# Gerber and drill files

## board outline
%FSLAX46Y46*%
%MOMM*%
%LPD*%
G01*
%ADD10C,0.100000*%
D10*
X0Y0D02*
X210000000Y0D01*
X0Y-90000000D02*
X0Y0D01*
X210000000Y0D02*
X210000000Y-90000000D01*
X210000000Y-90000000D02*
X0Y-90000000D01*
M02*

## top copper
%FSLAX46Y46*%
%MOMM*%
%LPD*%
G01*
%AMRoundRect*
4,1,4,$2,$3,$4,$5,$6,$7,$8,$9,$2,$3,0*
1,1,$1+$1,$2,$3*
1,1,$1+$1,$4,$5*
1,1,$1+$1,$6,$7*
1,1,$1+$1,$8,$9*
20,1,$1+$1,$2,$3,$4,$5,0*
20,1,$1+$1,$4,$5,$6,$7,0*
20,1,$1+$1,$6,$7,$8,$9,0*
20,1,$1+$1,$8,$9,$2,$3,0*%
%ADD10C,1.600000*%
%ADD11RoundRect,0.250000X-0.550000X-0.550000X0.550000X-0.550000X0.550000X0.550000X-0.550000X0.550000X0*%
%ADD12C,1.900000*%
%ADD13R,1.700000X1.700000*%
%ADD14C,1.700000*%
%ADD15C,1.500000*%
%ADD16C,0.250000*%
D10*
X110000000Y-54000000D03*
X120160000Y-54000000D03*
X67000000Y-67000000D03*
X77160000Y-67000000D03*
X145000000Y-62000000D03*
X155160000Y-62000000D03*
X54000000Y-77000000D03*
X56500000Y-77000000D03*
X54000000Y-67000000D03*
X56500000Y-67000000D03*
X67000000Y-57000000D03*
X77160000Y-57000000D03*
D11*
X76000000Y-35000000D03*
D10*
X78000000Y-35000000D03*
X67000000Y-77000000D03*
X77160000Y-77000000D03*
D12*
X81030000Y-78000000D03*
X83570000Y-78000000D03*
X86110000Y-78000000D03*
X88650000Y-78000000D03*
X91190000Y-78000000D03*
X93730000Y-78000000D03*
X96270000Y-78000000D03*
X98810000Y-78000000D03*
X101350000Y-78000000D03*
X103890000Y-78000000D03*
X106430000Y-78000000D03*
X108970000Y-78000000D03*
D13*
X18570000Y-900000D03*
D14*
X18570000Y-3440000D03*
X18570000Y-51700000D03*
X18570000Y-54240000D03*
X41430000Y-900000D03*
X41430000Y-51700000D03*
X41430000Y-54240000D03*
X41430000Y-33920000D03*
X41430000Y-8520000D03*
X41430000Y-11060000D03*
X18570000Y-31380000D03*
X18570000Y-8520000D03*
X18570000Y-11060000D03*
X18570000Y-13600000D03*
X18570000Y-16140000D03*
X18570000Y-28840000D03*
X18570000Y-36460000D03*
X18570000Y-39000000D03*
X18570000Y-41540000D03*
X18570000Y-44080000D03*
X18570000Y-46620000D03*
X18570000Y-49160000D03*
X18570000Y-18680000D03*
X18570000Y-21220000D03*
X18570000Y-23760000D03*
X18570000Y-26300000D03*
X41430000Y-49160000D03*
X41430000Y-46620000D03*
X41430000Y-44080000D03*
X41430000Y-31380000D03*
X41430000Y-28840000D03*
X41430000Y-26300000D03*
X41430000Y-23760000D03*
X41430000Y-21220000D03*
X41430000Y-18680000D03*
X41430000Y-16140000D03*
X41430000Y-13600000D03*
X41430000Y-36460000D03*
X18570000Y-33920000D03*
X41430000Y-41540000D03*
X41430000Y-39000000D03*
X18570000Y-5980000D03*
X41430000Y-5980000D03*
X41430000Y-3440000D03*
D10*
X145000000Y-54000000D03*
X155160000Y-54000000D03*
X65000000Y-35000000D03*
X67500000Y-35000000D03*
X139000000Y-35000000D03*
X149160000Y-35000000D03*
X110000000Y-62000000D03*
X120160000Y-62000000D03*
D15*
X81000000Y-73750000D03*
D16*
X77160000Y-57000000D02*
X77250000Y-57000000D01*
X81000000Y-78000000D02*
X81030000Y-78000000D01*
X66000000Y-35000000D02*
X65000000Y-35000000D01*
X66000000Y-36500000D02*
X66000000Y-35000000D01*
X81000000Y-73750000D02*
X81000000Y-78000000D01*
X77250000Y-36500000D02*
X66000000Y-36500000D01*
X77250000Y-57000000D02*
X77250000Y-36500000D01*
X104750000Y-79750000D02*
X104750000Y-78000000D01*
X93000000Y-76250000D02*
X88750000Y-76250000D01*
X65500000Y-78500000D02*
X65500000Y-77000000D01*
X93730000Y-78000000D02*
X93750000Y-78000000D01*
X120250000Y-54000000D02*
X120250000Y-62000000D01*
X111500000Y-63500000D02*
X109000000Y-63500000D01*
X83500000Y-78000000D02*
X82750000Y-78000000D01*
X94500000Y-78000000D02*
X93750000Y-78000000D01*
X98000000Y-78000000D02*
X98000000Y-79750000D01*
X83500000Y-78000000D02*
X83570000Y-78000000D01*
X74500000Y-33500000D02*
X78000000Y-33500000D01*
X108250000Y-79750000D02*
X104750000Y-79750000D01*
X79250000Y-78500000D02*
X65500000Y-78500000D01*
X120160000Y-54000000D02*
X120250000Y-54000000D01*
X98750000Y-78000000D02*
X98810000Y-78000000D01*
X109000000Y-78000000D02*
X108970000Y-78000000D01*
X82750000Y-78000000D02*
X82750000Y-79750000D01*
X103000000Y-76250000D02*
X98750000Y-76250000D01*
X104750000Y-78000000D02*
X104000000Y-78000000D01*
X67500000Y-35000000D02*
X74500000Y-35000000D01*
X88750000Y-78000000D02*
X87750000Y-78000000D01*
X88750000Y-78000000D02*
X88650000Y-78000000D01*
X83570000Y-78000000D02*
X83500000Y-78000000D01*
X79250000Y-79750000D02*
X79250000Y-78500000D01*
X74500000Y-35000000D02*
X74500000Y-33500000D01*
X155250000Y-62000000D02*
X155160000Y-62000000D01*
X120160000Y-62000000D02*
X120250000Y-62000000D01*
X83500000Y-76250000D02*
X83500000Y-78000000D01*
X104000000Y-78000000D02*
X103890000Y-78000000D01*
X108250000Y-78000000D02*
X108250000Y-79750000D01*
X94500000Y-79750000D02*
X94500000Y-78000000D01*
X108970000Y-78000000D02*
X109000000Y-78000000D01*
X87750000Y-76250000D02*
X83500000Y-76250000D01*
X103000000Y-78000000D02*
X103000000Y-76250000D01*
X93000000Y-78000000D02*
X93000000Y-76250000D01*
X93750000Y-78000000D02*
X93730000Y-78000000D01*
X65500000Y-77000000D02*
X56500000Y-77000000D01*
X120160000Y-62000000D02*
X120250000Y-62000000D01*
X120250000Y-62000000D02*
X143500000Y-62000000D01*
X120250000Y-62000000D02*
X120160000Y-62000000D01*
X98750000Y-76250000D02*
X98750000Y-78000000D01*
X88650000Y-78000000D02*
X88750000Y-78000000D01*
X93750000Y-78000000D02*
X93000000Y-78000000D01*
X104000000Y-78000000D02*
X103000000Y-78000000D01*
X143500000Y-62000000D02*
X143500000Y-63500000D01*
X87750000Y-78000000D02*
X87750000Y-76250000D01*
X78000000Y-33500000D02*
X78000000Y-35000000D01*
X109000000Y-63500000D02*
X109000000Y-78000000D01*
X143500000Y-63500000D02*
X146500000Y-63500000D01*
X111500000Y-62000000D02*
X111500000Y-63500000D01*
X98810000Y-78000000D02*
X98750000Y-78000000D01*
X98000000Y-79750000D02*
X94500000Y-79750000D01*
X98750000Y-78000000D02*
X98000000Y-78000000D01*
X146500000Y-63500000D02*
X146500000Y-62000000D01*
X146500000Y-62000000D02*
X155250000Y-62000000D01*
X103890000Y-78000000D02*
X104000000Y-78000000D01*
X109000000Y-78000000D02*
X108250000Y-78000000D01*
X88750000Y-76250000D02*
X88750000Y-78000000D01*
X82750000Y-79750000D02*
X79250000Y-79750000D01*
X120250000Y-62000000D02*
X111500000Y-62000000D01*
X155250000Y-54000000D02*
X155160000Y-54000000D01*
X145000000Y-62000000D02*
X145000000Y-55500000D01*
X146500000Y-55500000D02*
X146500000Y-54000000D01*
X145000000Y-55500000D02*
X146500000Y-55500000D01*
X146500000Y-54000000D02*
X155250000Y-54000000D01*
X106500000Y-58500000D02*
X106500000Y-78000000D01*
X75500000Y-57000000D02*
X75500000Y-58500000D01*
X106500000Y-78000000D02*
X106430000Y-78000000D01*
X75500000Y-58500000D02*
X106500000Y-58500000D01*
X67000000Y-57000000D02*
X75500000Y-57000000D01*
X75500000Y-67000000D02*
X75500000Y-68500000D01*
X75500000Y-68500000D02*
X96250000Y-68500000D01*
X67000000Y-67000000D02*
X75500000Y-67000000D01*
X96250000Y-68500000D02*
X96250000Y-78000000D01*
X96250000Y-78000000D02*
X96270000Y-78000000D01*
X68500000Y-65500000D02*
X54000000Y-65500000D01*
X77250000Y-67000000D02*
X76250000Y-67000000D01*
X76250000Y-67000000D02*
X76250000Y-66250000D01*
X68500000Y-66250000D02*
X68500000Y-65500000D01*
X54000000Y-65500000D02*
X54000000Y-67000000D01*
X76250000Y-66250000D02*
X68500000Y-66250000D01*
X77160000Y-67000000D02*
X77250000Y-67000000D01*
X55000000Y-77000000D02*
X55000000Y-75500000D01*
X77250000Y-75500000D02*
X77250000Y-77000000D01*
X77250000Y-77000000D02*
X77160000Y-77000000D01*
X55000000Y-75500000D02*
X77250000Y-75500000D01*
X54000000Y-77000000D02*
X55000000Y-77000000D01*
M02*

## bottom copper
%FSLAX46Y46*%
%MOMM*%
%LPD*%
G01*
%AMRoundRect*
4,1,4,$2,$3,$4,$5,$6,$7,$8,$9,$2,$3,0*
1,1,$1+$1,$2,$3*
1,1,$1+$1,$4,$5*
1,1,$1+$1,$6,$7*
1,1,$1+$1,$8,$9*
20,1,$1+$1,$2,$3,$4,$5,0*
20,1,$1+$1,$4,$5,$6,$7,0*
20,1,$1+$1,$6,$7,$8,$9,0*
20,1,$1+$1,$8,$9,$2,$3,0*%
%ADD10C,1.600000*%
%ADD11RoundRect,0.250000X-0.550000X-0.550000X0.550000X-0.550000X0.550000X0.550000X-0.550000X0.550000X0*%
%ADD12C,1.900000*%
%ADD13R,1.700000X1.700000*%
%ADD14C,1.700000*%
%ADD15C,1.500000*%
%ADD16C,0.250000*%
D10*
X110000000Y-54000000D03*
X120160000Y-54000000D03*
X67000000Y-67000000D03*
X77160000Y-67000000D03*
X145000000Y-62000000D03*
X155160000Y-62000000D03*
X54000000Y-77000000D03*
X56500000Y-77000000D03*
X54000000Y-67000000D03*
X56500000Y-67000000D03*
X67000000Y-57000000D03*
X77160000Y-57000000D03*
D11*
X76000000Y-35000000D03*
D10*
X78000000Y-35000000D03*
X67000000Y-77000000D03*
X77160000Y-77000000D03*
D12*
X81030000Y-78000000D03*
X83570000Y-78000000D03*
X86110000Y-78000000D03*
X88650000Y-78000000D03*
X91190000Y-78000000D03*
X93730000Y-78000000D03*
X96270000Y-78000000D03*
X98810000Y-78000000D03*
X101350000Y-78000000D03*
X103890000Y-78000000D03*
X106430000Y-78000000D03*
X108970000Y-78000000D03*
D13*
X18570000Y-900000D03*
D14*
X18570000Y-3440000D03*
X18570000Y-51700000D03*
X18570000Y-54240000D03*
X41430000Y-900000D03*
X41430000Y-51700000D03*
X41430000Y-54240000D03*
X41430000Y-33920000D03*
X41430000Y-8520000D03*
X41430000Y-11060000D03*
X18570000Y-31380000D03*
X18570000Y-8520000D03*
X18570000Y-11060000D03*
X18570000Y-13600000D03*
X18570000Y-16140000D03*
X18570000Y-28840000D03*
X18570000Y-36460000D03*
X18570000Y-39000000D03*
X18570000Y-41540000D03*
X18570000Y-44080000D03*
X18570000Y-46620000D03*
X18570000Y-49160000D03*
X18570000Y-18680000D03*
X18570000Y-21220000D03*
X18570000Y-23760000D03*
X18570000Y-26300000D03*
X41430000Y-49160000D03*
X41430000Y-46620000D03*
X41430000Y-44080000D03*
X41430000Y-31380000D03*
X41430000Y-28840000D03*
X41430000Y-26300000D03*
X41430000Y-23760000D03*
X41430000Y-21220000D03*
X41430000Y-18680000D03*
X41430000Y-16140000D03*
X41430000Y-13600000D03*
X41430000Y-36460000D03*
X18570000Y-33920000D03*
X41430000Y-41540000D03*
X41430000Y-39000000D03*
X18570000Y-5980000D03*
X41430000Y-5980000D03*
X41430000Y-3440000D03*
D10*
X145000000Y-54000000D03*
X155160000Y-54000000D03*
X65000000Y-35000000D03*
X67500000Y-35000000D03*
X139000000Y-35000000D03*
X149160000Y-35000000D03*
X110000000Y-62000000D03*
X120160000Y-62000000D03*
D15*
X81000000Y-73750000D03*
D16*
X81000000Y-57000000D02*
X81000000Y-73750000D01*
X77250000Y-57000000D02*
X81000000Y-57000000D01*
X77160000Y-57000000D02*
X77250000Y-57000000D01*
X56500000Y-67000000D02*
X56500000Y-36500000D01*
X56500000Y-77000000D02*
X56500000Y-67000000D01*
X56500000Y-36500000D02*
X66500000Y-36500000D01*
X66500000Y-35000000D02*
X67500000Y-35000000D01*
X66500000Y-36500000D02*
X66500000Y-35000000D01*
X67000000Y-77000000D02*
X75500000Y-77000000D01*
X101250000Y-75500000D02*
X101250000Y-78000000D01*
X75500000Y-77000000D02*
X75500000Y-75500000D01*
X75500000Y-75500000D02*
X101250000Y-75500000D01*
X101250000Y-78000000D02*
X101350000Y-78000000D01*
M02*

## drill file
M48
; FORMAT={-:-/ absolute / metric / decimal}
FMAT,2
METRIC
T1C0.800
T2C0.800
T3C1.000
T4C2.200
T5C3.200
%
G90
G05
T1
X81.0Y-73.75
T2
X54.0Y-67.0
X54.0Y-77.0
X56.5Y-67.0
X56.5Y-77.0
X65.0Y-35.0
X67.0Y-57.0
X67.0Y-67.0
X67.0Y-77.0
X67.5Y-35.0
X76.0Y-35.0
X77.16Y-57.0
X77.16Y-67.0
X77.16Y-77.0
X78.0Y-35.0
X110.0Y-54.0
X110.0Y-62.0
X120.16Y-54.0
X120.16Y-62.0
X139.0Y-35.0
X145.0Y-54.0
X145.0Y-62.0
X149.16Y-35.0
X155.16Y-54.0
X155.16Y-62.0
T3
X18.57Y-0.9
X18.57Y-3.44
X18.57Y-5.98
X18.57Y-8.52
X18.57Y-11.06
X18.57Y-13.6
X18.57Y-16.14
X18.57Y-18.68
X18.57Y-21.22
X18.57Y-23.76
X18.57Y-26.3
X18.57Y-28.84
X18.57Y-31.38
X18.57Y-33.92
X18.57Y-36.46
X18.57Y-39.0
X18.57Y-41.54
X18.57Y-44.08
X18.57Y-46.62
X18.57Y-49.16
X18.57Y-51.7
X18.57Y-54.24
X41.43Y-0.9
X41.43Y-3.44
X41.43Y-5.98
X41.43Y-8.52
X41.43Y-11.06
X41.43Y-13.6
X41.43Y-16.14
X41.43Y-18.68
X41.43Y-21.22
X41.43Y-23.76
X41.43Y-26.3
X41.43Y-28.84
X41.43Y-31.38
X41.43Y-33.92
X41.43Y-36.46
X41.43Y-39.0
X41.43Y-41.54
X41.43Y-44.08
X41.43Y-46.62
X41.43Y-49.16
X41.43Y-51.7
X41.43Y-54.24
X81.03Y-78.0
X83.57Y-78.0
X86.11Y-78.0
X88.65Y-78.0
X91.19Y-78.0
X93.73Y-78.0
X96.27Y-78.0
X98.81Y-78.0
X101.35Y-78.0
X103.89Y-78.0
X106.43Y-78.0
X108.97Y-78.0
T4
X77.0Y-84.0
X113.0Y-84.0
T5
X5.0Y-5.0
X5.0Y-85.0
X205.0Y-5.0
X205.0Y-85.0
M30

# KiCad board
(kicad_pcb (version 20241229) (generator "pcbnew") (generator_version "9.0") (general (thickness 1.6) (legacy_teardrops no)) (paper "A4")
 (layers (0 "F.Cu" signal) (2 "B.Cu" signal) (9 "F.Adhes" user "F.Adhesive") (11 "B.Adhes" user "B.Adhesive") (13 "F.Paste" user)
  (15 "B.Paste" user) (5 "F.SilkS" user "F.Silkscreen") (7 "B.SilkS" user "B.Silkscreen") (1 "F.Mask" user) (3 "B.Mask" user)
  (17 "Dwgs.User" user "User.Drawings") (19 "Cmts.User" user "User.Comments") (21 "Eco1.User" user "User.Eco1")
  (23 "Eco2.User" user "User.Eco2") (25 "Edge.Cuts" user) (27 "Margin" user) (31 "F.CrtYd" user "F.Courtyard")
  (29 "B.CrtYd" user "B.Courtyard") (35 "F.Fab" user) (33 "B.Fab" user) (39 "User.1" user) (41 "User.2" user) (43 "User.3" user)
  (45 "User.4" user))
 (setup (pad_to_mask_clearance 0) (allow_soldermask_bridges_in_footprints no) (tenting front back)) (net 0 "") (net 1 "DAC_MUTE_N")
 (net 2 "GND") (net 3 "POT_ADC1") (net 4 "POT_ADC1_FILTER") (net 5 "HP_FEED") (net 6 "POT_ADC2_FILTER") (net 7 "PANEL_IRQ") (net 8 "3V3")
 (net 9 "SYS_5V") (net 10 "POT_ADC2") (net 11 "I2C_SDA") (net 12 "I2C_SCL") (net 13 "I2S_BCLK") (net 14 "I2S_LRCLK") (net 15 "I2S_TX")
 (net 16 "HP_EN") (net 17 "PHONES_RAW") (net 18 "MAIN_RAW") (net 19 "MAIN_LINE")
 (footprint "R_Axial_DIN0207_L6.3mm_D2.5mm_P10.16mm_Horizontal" (layer "F.Cu") (at 110 54)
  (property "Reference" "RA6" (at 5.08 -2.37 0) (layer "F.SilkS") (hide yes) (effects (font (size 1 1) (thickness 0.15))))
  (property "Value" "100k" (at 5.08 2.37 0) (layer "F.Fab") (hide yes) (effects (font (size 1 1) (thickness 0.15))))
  (pad "1" thru_hole circle (at 0 0) (size 1.6 1.6) (drill 0.8) (layers "*.Cu" "*.Mask") (remove_unused_layers no) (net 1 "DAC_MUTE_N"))
  (pad "2" thru_hole circle (at 10.16 0) (size 1.6 1.6) (drill 0.8) (layers "*.Cu" "*.Mask") (remove_unused_layers no) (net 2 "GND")))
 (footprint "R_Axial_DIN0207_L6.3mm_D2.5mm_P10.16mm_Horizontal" (layer "F.Cu") (at 67 67)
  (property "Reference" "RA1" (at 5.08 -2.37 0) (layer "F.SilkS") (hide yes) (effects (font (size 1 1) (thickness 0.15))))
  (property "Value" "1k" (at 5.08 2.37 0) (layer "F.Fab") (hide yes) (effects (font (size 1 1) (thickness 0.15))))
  (pad "1" thru_hole circle (at 0 0) (size 1.6 1.6) (drill 0.8) (layers "*.Cu" "*.Mask") (remove_unused_layers no) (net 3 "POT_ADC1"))
  (pad "2" thru_hole circle (at 10.16 0) (size 1.6 1.6) (drill 0.8) (layers "*.Cu" "*.Mask") (remove_unused_layers no)
   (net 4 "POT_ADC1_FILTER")))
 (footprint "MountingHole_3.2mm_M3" (layer "F.Cu") (at 5 5)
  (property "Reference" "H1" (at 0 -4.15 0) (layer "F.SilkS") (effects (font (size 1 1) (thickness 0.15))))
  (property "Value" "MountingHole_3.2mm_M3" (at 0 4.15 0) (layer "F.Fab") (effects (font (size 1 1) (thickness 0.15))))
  (pad "" np_thru_hole circle (at 0 0) (size 3.2 3.2) (drill 3.2) (layers "*.Cu" "*.Mask")))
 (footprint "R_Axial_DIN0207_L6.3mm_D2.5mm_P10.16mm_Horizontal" (layer "F.Cu") (at 145 62)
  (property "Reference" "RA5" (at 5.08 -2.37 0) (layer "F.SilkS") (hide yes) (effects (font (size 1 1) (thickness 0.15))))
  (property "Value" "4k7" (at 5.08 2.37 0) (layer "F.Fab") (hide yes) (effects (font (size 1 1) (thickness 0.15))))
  (pad "1" thru_hole circle (at 0 0) (size 1.6 1.6) (drill 0.8) (layers "*.Cu" "*.Mask") (remove_unused_layers no) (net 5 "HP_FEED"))
  (pad "2" thru_hole circle (at 10.16 0) (size 1.6 1.6) (drill 0.8) (layers "*.Cu" "*.Mask") (remove_unused_layers no) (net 2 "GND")))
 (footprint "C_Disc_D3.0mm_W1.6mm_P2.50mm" (layer "F.Cu") (at 54 77)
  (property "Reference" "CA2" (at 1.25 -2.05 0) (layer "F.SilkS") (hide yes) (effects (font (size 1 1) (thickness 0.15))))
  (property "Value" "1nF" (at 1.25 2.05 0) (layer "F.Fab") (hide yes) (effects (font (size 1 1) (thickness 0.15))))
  (pad "1" thru_hole circle (at 0 0) (size 1.6 1.6) (drill 0.8) (layers "*.Cu" "*.Mask") (remove_unused_layers no) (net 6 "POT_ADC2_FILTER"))
  (pad "2" thru_hole circle (at 2.5 0) (size 1.6 1.6) (drill 0.8) (layers "*.Cu" "*.Mask") (remove_unused_layers no) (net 2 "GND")))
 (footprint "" (layer "F.Cu") (at 112 42)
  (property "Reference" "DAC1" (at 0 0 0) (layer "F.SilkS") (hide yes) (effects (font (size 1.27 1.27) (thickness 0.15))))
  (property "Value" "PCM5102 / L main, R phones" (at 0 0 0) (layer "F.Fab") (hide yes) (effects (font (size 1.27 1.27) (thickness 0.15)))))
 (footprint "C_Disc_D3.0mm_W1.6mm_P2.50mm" (layer "F.Cu") (at 54 67)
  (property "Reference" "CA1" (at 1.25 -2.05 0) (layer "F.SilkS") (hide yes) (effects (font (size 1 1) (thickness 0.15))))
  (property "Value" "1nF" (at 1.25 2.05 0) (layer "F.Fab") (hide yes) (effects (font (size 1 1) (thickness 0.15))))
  (pad "1" thru_hole circle (at 0 0) (size 1.6 1.6) (drill 0.8) (layers "*.Cu" "*.Mask") (remove_unused_layers no) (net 4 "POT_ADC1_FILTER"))
  (pad "2" thru_hole circle (at 2.5 0) (size 1.6 1.6) (drill 0.8) (layers "*.Cu" "*.Mask") (remove_unused_layers no) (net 2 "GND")))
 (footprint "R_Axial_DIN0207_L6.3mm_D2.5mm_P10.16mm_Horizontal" (layer "F.Cu") (at 67 57)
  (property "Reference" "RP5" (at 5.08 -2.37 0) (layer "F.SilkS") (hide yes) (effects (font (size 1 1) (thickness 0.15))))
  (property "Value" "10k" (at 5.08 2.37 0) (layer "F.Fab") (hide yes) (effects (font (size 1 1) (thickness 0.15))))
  (pad "1" thru_hole circle (at 0 0) (size 1.6 1.6) (drill 0.8) (layers "*.Cu" "*.Mask") (remove_unused_layers no) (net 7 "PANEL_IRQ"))
  (pad "2" thru_hole circle (at 10.16 0) (size 1.6 1.6) (drill 0.8) (layers "*.Cu" "*.Mask") (remove_unused_layers no) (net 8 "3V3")))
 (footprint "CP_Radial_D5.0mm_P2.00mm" (layer "F.Cu") (at 76 35)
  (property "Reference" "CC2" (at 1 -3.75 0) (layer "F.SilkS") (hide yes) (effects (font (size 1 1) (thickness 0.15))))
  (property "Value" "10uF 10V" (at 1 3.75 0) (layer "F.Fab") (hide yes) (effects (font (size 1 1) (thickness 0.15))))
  (pad "1" thru_hole roundrect (at 0 0) (size 1.6 1.6) (drill 0.8) (layers "*.Cu" "*.Mask") (remove_unused_layers no)
   (roundrect_rratio 0.15625) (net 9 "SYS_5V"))
  (pad "2" thru_hole circle (at 2 0) (size 1.6 1.6) (drill 0.8) (layers "*.Cu" "*.Mask") (remove_unused_layers no) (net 2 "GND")))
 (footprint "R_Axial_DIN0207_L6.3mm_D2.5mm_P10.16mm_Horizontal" (layer "F.Cu") (at 67 77)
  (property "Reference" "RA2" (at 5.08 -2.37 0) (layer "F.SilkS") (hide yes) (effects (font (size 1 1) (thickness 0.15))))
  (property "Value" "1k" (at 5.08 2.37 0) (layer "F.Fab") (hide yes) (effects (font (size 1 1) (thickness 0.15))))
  (pad "1" thru_hole circle (at 0 0) (size 1.6 1.6) (drill 0.8) (layers "*.Cu" "*.Mask") (remove_unused_layers no) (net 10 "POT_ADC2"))
  (pad "2" thru_hole circle (at 10.16 0) (size 1.6 1.6) (drill 0.8) (layers "*.Cu" "*.Mask") (remove_unused_layers no)
   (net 6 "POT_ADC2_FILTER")))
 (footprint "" (layer "F.Cu") (at 174 13)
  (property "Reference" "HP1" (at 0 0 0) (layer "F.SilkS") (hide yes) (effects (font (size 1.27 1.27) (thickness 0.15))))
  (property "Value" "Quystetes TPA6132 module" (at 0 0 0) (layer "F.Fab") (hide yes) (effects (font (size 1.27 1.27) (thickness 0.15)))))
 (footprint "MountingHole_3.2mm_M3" (layer "F.Cu") (at 205 5)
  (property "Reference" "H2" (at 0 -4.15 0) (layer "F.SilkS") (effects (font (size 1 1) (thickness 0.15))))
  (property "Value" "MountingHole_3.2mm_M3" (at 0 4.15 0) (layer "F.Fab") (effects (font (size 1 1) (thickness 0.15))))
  (pad "" np_thru_hole circle (at 0 0) (size 3.2 3.2) (drill 3.2) (layers "*.Cu" "*.Mask")))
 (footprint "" (layer "F.Cu") (at 95 78)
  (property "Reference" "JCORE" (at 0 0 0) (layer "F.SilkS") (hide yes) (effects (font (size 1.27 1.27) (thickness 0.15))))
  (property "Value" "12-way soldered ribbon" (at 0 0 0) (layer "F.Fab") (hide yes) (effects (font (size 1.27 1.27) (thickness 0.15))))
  (pad "1" thru_hole circle (at -13.97 0) (size 1.9 1.9) (drill 1) (layers "*.Cu") (remove_unused_layers no) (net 8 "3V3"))
  (pad "2" thru_hole circle (at -11.43 0) (size 1.9 1.9) (drill 1) (layers "*.Cu") (remove_unused_layers no) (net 2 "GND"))
  (pad "3" thru_hole circle (at -8.89 0) (size 1.9 1.9) (drill 1) (layers "*.Cu") (remove_unused_layers no) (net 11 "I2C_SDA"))
  (pad "4" thru_hole circle (at -6.35 0) (size 1.9 1.9) (drill 1) (layers "*.Cu") (remove_unused_layers no) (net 2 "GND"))
  (pad "5" thru_hole circle (at -3.81 0) (size 1.9 1.9) (drill 1) (layers "*.Cu") (remove_unused_layers no) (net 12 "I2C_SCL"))
  (pad "6" thru_hole circle (at -1.27 0) (size 1.9 1.9) (drill 1) (layers "*.Cu") (remove_unused_layers no) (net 2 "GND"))
  (pad "7" thru_hole circle (at 1.27 0) (size 1.9 1.9) (drill 1) (layers "*.Cu") (remove_unused_layers no) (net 3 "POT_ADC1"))
  (pad "8" thru_hole circle (at 3.81 0) (size 1.9 1.9) (drill 1) (layers "*.Cu") (remove_unused_layers no) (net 2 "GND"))
  (pad "9" thru_hole circle (at 6.35 0) (size 1.9 1.9) (drill 1) (layers "*.Cu") (remove_unused_layers no) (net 10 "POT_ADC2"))
  (pad "10" thru_hole circle (at 8.89 0) (size 1.9 1.9) (drill 1) (layers "*.Cu") (remove_unused_layers no) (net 2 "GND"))
  (pad "11" thru_hole circle (at 11.43 0) (size 1.9 1.9) (drill 1) (layers "*.Cu") (remove_unused_layers no) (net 7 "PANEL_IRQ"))
  (pad "12" thru_hole circle (at 13.97 0) (size 1.9 1.9) (drill 1) (layers "*.Cu") (remove_unused_layers no) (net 2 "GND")))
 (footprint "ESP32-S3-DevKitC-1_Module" (layer "F.Cu") (at 30 31)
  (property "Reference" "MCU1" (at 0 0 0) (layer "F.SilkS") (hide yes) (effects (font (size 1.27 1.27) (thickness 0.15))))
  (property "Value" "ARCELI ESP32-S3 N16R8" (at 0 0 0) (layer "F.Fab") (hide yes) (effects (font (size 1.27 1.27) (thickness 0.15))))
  (pad "3V3" thru_hole rect (at -11.43 -30.1) (size 1.7 1.7) (drill 1) (layers "*.Cu" "*.Mask") (remove_unused_layers no) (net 8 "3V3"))
  (pad "3V3" thru_hole circle (at -11.43 -27.56) (size 1.7 1.7) (drill 1) (layers "*.Cu" "*.Mask") (remove_unused_layers no) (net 8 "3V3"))
  (pad "5V" thru_hole circle (at -11.43 20.7) (size 1.7 1.7) (drill 1) (layers "*.Cu" "*.Mask") (remove_unused_layers no) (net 9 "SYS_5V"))
  (pad "GND" thru_hole circle (at -11.43 23.24) (size 1.7 1.7) (drill 1) (layers "*.Cu" "*.Mask") (remove_unused_layers no) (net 2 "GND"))
  (pad "GND" thru_hole circle (at 11.43 -30.1) (size 1.7 1.7) (drill 1) (layers "*.Cu" "*.Mask") (remove_unused_layers no) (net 2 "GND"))
  (pad "GND" thru_hole circle (at 11.43 20.7) (size 1.7 1.7) (drill 1) (layers "*.Cu" "*.Mask") (remove_unused_layers no) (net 2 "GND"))
  (pad "GND" thru_hole circle (at 11.43 23.24) (size 1.7 1.7) (drill 1) (layers "*.Cu" "*.Mask") (remove_unused_layers no) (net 2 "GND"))
  (pad "GPIO0" thru_hole circle (at 11.43 2.92) (size 1.7 1.7) (drill 1) (layers "*.Cu" "*.Mask") (remove_unused_layers no))
  (pad "GPIO1" thru_hole circle (at 11.43 -22.48) (size 1.7 1.7) (drill 1) (layers "*.Cu" "*.Mask") (remove_unused_layers no)
   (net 11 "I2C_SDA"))
  (pad "GPIO2" thru_hole circle (at 11.43 -19.94) (size 1.7 1.7) (drill 1) (layers "*.Cu" "*.Mask") (remove_unused_layers no)
   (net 12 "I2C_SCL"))
  (pad "GPIO3" thru_hole circle (at -11.43 0.38) (size 1.7 1.7) (drill 1) (layers "*.Cu" "*.Mask") (remove_unused_layers no))
  (pad "GPIO4" thru_hole circle (at -11.43 -22.48) (size 1.7 1.7) (drill 1) (layers "*.Cu" "*.Mask") (remove_unused_layers no)
   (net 4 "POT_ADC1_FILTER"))
  (pad "GPIO5" thru_hole circle (at -11.43 -19.94) (size 1.7 1.7) (drill 1) (layers "*.Cu" "*.Mask") (remove_unused_layers no)
   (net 6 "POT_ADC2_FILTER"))
  (pad "GPIO6" thru_hole circle (at -11.43 -17.4) (size 1.7 1.7) (drill 1) (layers "*.Cu" "*.Mask") (remove_unused_layers no))
  (pad "GPIO7" thru_hole circle (at -11.43 -14.86) (size 1.7 1.7) (drill 1) (layers "*.Cu" "*.Mask") (remove_unused_layers no))
  (pad "GPIO8" thru_hole circle (at -11.43 -2.16) (size 1.7 1.7) (drill 1) (layers "*.Cu" "*.Mask") (remove_unused_layers no))
  (pad "GPIO9" thru_hole circle (at -11.43 5.46) (size 1.7 1.7) (drill 1) (layers "*.Cu" "*.Mask") (remove_unused_layers no))
  (pad "GPIO10" thru_hole circle (at -11.43 8) (size 1.7 1.7) (drill 1) (layers "*.Cu" "*.Mask") (remove_unused_layers no)
   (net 7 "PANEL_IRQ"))
  (pad "GPIO11" thru_hole circle (at -11.43 10.54) (size 1.7 1.7) (drill 1) (layers "*.Cu" "*.Mask") (remove_unused_layers no))
  (pad "GPIO12" thru_hole circle (at -11.43 13.08) (size 1.7 1.7) (drill 1) (layers "*.Cu" "*.Mask") (remove_unused_layers no))
  (pad "GPIO13" thru_hole circle (at -11.43 15.62) (size 1.7 1.7) (drill 1) (layers "*.Cu" "*.Mask") (remove_unused_layers no))
  (pad "GPIO14" thru_hole circle (at -11.43 18.16) (size 1.7 1.7) (drill 1) (layers "*.Cu" "*.Mask") (remove_unused_layers no))
  (pad "GPIO15" thru_hole circle (at -11.43 -12.32) (size 1.7 1.7) (drill 1) (layers "*.Cu" "*.Mask") (remove_unused_layers no)
   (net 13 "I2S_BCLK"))
  (pad "GPIO16" thru_hole circle (at -11.43 -9.78) (size 1.7 1.7) (drill 1) (layers "*.Cu" "*.Mask") (remove_unused_layers no)
   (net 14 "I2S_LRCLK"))
  (pad "GPIO17" thru_hole circle (at -11.43 -7.24) (size 1.7 1.7) (drill 1) (layers "*.Cu" "*.Mask") (remove_unused_layers no)
   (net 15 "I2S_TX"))
  (pad "GPIO18" thru_hole circle (at -11.43 -4.7) (size 1.7 1.7) (drill 1) (layers "*.Cu" "*.Mask") (remove_unused_layers no))
  (pad "GPIO19" thru_hole circle (at 11.43 18.16) (size 1.7 1.7) (drill 1) (layers "*.Cu" "*.Mask") (remove_unused_layers no))
  (pad "GPIO20" thru_hole circle (at 11.43 15.62) (size 1.7 1.7) (drill 1) (layers "*.Cu" "*.Mask") (remove_unused_layers no))
  (pad "GPIO21" thru_hole circle (at 11.43 13.08) (size 1.7 1.7) (drill 1) (layers "*.Cu" "*.Mask") (remove_unused_layers no))
  (pad "GPIO35" thru_hole circle (at 11.43 0.38) (size 1.7 1.7) (drill 1) (layers "*.Cu" "*.Mask") (remove_unused_layers no))
  (pad "GPIO36" thru_hole circle (at 11.43 -2.16) (size 1.7 1.7) (drill 1) (layers "*.Cu" "*.Mask") (remove_unused_layers no))
  (pad "GPIO37" thru_hole circle (at 11.43 -4.7) (size 1.7 1.7) (drill 1) (layers "*.Cu" "*.Mask") (remove_unused_layers no))
  (pad "GPIO38" thru_hole circle (at 11.43 -7.24) (size 1.7 1.7) (drill 1) (layers "*.Cu" "*.Mask") (remove_unused_layers no))
  (pad "GPIO39" thru_hole circle (at 11.43 -9.78) (size 1.7 1.7) (drill 1) (layers "*.Cu" "*.Mask") (remove_unused_layers no))
  (pad "GPIO40" thru_hole circle (at 11.43 -12.32) (size 1.7 1.7) (drill 1) (layers "*.Cu" "*.Mask") (remove_unused_layers no)
   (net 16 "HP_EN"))
  (pad "GPIO41" thru_hole circle (at 11.43 -14.86) (size 1.7 1.7) (drill 1) (layers "*.Cu" "*.Mask") (remove_unused_layers no)
   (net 1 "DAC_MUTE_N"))
  (pad "GPIO42" thru_hole circle (at 11.43 -17.4) (size 1.7 1.7) (drill 1) (layers "*.Cu" "*.Mask") (remove_unused_layers no))
  (pad "GPIO45" thru_hole circle (at 11.43 5.46) (size 1.7 1.7) (drill 1) (layers "*.Cu" "*.Mask") (remove_unused_layers no))
  (pad "GPIO46" thru_hole circle (at -11.43 2.92) (size 1.7 1.7) (drill 1) (layers "*.Cu" "*.Mask") (remove_unused_layers no))
  (pad "GPIO47" thru_hole circle (at 11.43 10.54) (size 1.7 1.7) (drill 1) (layers "*.Cu" "*.Mask") (remove_unused_layers no))
  (pad "GPIO48" thru_hole circle (at 11.43 8) (size 1.7 1.7) (drill 1) (layers "*.Cu" "*.Mask") (remove_unused_layers no))
  (pad "RST" thru_hole circle (at -11.43 -25.02) (size 1.7 1.7) (drill 1) (layers "*.Cu" "*.Mask") (remove_unused_layers no))
  (pad "RX" thru_hole circle (at 11.43 -25.02) (size 1.7 1.7) (drill 1) (layers "*.Cu" "*.Mask") (remove_unused_layers no))
  (pad "TX" thru_hole circle (at 11.43 -27.56) (size 1.7 1.7) (drill 1) (layers "*.Cu" "*.Mask") (remove_unused_layers no)))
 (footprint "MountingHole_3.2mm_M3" (layer "F.Cu") (at 5 85)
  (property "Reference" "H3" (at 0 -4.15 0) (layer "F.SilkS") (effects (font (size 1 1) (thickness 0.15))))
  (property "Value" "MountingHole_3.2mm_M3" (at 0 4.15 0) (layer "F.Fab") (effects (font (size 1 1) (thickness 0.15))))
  (pad "" np_thru_hole circle (at 0 0) (size 3.2 3.2) (drill 3.2) (layers "*.Cu" "*.Mask")))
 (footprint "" (layer "F.Cu") (at 144 5)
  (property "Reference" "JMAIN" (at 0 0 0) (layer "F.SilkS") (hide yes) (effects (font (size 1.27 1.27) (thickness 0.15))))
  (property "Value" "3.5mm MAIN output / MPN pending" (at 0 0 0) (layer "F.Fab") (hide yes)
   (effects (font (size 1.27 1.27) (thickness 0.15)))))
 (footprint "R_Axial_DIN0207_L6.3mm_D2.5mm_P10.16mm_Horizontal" (layer "F.Cu") (at 145 54)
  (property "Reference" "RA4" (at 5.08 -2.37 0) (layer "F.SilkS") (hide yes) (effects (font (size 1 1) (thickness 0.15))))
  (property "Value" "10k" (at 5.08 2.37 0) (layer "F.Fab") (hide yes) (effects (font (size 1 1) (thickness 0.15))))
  (pad "1" thru_hole circle (at 0 0) (size 1.6 1.6) (drill 0.8) (layers "*.Cu" "*.Mask") (remove_unused_layers no) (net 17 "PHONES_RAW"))
  (pad "2" thru_hole circle (at 10.16 0) (size 1.6 1.6) (drill 0.8) (layers "*.Cu" "*.Mask") (remove_unused_layers no) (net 5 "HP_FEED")))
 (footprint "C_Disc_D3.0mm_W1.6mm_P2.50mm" (layer "F.Cu") (at 65 35)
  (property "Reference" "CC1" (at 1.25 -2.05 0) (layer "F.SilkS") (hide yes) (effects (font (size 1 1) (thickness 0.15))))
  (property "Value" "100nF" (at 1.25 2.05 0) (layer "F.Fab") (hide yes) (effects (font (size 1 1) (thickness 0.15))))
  (pad "1" thru_hole circle (at 0 0) (size 1.6 1.6) (drill 0.8) (layers "*.Cu" "*.Mask") (remove_unused_layers no) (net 8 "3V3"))
  (pad "2" thru_hole circle (at 2.5 0) (size 1.6 1.6) (drill 0.8) (layers "*.Cu" "*.Mask") (remove_unused_layers no) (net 2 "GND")))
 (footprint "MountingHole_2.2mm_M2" (layer "F.Cu") (at 77 84)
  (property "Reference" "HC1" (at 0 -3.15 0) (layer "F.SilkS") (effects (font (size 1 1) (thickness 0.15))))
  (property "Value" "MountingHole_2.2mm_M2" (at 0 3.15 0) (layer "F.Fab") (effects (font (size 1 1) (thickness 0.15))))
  (pad "" np_thru_hole circle (at 0 0) (size 2.2 2.2) (drill 2.2) (layers "*.Cu" "*.Mask")))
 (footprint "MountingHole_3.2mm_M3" (layer "F.Cu") (at 205 85)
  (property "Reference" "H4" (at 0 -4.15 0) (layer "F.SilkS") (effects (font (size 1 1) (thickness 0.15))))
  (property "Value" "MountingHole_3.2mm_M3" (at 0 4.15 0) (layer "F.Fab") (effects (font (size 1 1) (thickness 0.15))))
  (pad "" np_thru_hole circle (at 0 0) (size 3.2 3.2) (drill 3.2) (layers "*.Cu" "*.Mask")))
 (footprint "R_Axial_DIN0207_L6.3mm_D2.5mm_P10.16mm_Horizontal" (layer "F.Cu") (at 139 35)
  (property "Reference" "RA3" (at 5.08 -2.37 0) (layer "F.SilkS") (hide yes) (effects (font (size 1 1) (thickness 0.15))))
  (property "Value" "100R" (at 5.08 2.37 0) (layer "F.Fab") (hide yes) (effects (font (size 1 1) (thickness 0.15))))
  (pad "1" thru_hole circle (at 0 0) (size 1.6 1.6) (drill 0.8) (layers "*.Cu" "*.Mask") (remove_unused_layers no) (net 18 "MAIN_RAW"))
  (pad "2" thru_hole circle (at 10.16 0) (size 1.6 1.6) (drill 0.8) (layers "*.Cu" "*.Mask") (remove_unused_layers no) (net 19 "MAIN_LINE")))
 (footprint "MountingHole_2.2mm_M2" (layer "F.Cu") (at 113 84)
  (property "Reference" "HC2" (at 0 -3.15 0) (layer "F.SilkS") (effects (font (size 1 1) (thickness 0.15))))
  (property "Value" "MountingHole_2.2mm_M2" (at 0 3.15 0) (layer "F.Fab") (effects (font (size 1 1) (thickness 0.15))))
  (pad "" np_thru_hole circle (at 0 0) (size 2.2 2.2) (drill 2.2) (layers "*.Cu" "*.Mask")))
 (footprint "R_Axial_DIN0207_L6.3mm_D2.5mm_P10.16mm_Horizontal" (layer "F.Cu") (at 110 62)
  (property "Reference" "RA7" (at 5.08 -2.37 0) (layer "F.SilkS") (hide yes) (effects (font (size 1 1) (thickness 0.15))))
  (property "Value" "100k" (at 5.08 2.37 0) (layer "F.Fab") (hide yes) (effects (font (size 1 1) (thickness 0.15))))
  (pad "1" thru_hole circle (at 0 0) (size 1.6 1.6) (drill 0.8) (layers "*.Cu" "*.Mask") (remove_unused_layers no) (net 16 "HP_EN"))
  (pad "2" thru_hole circle (at 10.16 0) (size 1.6 1.6) (drill 0.8) (layers "*.Cu" "*.Mask") (remove_unused_layers no) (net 2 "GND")))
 (gr_line (start 0 0) (end 210 0) (stroke (width 0.1) (type default)) (layer "Edge.Cuts"))
 (gr_line (start 0 90) (end 0 0) (stroke (width 0.1) (type default)) (layer "Edge.Cuts"))
 (gr_line (start 210 0) (end 210 90) (stroke (width 0.1) (type default)) (layer "Edge.Cuts"))
 (gr_line (start 210 90) (end 0 90) (stroke (width 0.1) (type default)) (layer "Edge.Cuts"))
 (segment (start 77.16 57) (end 77.25 57) (width 0.25) (layer "F.Cu") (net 8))
 (segment (start 81 78) (end 81.03 78) (width 0.25) (layer "F.Cu") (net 8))
 (segment (start 66 35) (end 65 35) (width 0.25) (layer "F.Cu") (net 8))
 (segment (start 66 36.5) (end 66 35) (width 0.25) (layer "F.Cu") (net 8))
 (segment (start 81 73.75) (end 81 78) (width 0.25) (layer "F.Cu") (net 8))
 (segment (start 77.25 36.5) (end 66 36.5) (width 0.25) (layer "F.Cu") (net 8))
 (segment (start 77.25 57) (end 77.25 36.5) (width 0.25) (layer "F.Cu") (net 8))
 (via (at 81 73.75) (size 1.5) (drill 0.8) (layers "F.Cu" "B.Cu") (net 8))
 (segment (start 81 57) (end 81 73.75) (width 0.25) (layer "B.Cu") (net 8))
 (segment (start 77.25 57) (end 81 57) (width 0.25) (layer "B.Cu") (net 8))
 (segment (start 77.16 57) (end 77.25 57) (width 0.25) (layer "B.Cu") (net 8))
 (segment (start 104.75 79.75) (end 104.75 78) (width 0.25) (layer "F.Cu") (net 2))
 (segment (start 93 76.25) (end 88.75 76.25) (width 0.25) (layer "F.Cu") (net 2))
 (segment (start 65.5 78.5) (end 65.5 77) (width 0.25) (layer "F.Cu") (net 2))
 (segment (start 93.73 78) (end 93.75 78) (width 0.25) (layer "F.Cu") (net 2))
 (segment (start 120.25 54) (end 120.25 62) (width 0.25) (layer "F.Cu") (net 2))
 (segment (start 111.5 63.5) (end 109 63.5) (width 0.25) (layer "F.Cu") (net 2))
 (segment (start 83.5 78) (end 82.75 78) (width 0.25) (layer "F.Cu") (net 2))
 (segment (start 94.5 78) (end 93.75 78) (width 0.25) (layer "F.Cu") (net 2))
 (segment (start 98 78) (end 98 79.75) (width 0.25) (layer "F.Cu") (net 2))
 (segment (start 83.5 78) (end 83.57 78) (width 0.25) (layer "F.Cu") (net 2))
 (segment (start 74.5 33.5) (end 78 33.5) (width 0.25) (layer "F.Cu") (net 2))
 (segment (start 108.25 79.75) (end 104.75 79.75) (width 0.25) (layer "F.Cu") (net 2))
 (segment (start 79.25 78.5) (end 65.5 78.5) (width 0.25) (layer "F.Cu") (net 2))
 (segment (start 120.16 54) (end 120.25 54) (width 0.25) (layer "F.Cu") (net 2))
 (segment (start 98.75 78) (end 98.81 78) (width 0.25) (layer "F.Cu") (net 2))
 (segment (start 109 78) (end 108.97 78) (width 0.25) (layer "F.Cu") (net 2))
 (segment (start 82.75 78) (end 82.75 79.75) (width 0.25) (layer "F.Cu") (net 2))
 (segment (start 103 76.25) (end 98.75 76.25) (width 0.25) (layer "F.Cu") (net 2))
 (segment (start 104.75 78) (end 104 78) (width 0.25) (layer "F.Cu") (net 2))
 (segment (start 67.5 35) (end 74.5 35) (width 0.25) (layer "F.Cu") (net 2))
 (segment (start 88.75 78) (end 87.75 78) (width 0.25) (layer "F.Cu") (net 2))
 (segment (start 88.75 78) (end 88.65 78) (width 0.25) (layer "F.Cu") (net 2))
 (segment (start 83.57 78) (end 83.5 78) (width 0.25) (layer "F.Cu") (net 2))
 (segment (start 79.25 79.75) (end 79.25 78.5) (width 0.25) (layer "F.Cu") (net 2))
 (segment (start 74.5 35) (end 74.5 33.5) (width 0.25) (layer "F.Cu") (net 2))
 (segment (start 155.25 62) (end 155.16 62) (width 0.25) (layer "F.Cu") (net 2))
 (segment (start 120.16 62) (end 120.25 62) (width 0.25) (layer "F.Cu") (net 2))
 (segment (start 83.5 76.25) (end 83.5 78) (width 0.25) (layer "F.Cu") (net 2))
 (segment (start 104 78) (end 103.89 78) (width 0.25) (layer "F.Cu") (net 2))
 (segment (start 108.25 78) (end 108.25 79.75) (width 0.25) (layer "F.Cu") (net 2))
 (segment (start 94.5 79.75) (end 94.5 78) (width 0.25) (layer "F.Cu") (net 2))
 (segment (start 108.97 78) (end 109 78) (width 0.25) (layer "F.Cu") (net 2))
 (segment (start 87.75 76.25) (end 83.5 76.25) (width 0.25) (layer "F.Cu") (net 2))
 (segment (start 103 78) (end 103 76.25) (width 0.25) (layer "F.Cu") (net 2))
 (segment (start 93 78) (end 93 76.25) (width 0.25) (layer "F.Cu") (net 2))
 (segment (start 93.75 78) (end 93.73 78) (width 0.25) (layer "F.Cu") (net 2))
 (segment (start 65.5 77) (end 56.5 77) (width 0.25) (layer "F.Cu") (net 2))
 (segment (start 120.16 62) (end 120.25 62) (width 0.25) (layer "F.Cu") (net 2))
 (segment (start 120.25 62) (end 143.5 62) (width 0.25) (layer "F.Cu") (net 2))
 (segment (start 120.25 62) (end 120.16 62) (width 0.25) (layer "F.Cu") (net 2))
 (segment (start 98.75 76.25) (end 98.75 78) (width 0.25) (layer "F.Cu") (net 2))
 (segment (start 88.65 78) (end 88.75 78) (width 0.25) (layer "F.Cu") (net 2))
 (segment (start 93.75 78) (end 93 78) (width 0.25) (layer "F.Cu") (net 2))
 (segment (start 104 78) (end 103 78) (width 0.25) (layer "F.Cu") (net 2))
 (segment (start 143.5 62) (end 143.5 63.5) (width 0.25) (layer "F.Cu") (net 2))
 (segment (start 87.75 78) (end 87.75 76.25) (width 0.25) (layer "F.Cu") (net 2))
 (segment (start 78 33.5) (end 78 35) (width 0.25) (layer "F.Cu") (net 2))
 (segment (start 109 63.5) (end 109 78) (width 0.25) (layer "F.Cu") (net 2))
 (segment (start 143.5 63.5) (end 146.5 63.5) (width 0.25) (layer "F.Cu") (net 2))
 (segment (start 111.5 62) (end 111.5 63.5) (width 0.25) (layer "F.Cu") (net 2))
 (segment (start 98.81 78) (end 98.75 78) (width 0.25) (layer "F.Cu") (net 2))
 (segment (start 98 79.75) (end 94.5 79.75) (width 0.25) (layer "F.Cu") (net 2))
 (segment (start 98.75 78) (end 98 78) (width 0.25) (layer "F.Cu") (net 2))
 (segment (start 146.5 63.5) (end 146.5 62) (width 0.25) (layer "F.Cu") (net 2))
 (segment (start 146.5 62) (end 155.25 62) (width 0.25) (layer "F.Cu") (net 2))
 (segment (start 103.89 78) (end 104 78) (width 0.25) (layer "F.Cu") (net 2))
 (segment (start 109 78) (end 108.25 78) (width 0.25) (layer "F.Cu") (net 2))
 (segment (start 88.75 76.25) (end 88.75 78) (width 0.25) (layer "F.Cu") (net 2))
 (segment (start 82.75 79.75) (end 79.25 79.75) (width 0.25) (layer "F.Cu") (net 2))
 (segment (start 120.25 62) (end 111.5 62) (width 0.25) (layer "F.Cu") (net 2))
 (segment (start 56.5 67) (end 56.5 36.5) (width 0.25) (layer "B.Cu") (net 2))
 (segment (start 56.5 77) (end 56.5 67) (width 0.25) (layer "B.Cu") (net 2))
 (segment (start 56.5 36.5) (end 66.5 36.5) (width 0.25) (layer "B.Cu") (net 2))
 (segment (start 66.5 35) (end 67.5 35) (width 0.25) (layer "B.Cu") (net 2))
 (segment (start 66.5 36.5) (end 66.5 35) (width 0.25) (layer "B.Cu") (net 2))
 (segment (start 155.25 54) (end 155.16 54) (width 0.25) (layer "F.Cu") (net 5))
 (segment (start 145 62) (end 145 55.5) (width 0.25) (layer "F.Cu") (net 5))
 (segment (start 146.5 55.5) (end 146.5 54) (width 0.25) (layer "F.Cu") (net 5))
 (segment (start 145 55.5) (end 146.5 55.5) (width 0.25) (layer "F.Cu") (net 5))
 (segment (start 146.5 54) (end 155.25 54) (width 0.25) (layer "F.Cu") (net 5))
 (segment (start 106.5 58.5) (end 106.5 78) (width 0.25) (layer "F.Cu") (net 7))
 (segment (start 75.5 57) (end 75.5 58.5) (width 0.25) (layer "F.Cu") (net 7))
 (segment (start 106.5 78) (end 106.43 78) (width 0.25) (layer "F.Cu") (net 7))
 (segment (start 75.5 58.5) (end 106.5 58.5) (width 0.25) (layer "F.Cu") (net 7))
 (segment (start 67 57) (end 75.5 57) (width 0.25) (layer "F.Cu") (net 7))
 (segment (start 75.5 67) (end 75.5 68.5) (width 0.25) (layer "F.Cu") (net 3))
 (segment (start 75.5 68.5) (end 96.25 68.5) (width 0.25) (layer "F.Cu") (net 3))
 (segment (start 67 67) (end 75.5 67) (width 0.25) (layer "F.Cu") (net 3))
 (segment (start 96.25 68.5) (end 96.25 78) (width 0.25) (layer "F.Cu") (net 3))
 (segment (start 96.25 78) (end 96.27 78) (width 0.25) (layer "F.Cu") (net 3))
 (segment (start 68.5 65.5) (end 54 65.5) (width 0.25) (layer "F.Cu") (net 4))
 (segment (start 77.25 67) (end 76.25 67) (width 0.25) (layer "F.Cu") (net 4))
 (segment (start 76.25 67) (end 76.25 66.25) (width 0.25) (layer "F.Cu") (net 4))
 (segment (start 68.5 66.25) (end 68.5 65.5) (width 0.25) (layer "F.Cu") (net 4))
 (segment (start 54 65.5) (end 54 67) (width 0.25) (layer "F.Cu") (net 4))
 (segment (start 76.25 66.25) (end 68.5 66.25) (width 0.25) (layer "F.Cu") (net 4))
 (segment (start 77.16 67) (end 77.25 67) (width 0.25) (layer "F.Cu") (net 4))
 (segment (start 67 77) (end 75.5 77) (width 0.25) (layer "B.Cu") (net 10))
 (segment (start 101.25 75.5) (end 101.25 78) (width 0.25) (layer "B.Cu") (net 10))
 (segment (start 75.5 77) (end 75.5 75.5) (width 0.25) (layer "B.Cu") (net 10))
 (segment (start 75.5 75.5) (end 101.25 75.5) (width 0.25) (layer "B.Cu") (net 10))
 (segment (start 101.25 78) (end 101.35 78) (width 0.25) (layer "B.Cu") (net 10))
 (segment (start 55 77) (end 55 75.5) (width 0.25) (layer "F.Cu") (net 6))
 (segment (start 77.25 75.5) (end 77.25 77) (width 0.25) (layer "F.Cu") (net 6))
 (segment (start 77.25 77) (end 77.16 77) (width 0.25) (layer "F.Cu") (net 6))
 (segment (start 55 75.5) (end 77.25 75.5) (width 0.25) (layer "F.Cu") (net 6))
 (segment (start 54 77) (end 55 77) (width 0.25) (layer "F.Cu") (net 6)))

